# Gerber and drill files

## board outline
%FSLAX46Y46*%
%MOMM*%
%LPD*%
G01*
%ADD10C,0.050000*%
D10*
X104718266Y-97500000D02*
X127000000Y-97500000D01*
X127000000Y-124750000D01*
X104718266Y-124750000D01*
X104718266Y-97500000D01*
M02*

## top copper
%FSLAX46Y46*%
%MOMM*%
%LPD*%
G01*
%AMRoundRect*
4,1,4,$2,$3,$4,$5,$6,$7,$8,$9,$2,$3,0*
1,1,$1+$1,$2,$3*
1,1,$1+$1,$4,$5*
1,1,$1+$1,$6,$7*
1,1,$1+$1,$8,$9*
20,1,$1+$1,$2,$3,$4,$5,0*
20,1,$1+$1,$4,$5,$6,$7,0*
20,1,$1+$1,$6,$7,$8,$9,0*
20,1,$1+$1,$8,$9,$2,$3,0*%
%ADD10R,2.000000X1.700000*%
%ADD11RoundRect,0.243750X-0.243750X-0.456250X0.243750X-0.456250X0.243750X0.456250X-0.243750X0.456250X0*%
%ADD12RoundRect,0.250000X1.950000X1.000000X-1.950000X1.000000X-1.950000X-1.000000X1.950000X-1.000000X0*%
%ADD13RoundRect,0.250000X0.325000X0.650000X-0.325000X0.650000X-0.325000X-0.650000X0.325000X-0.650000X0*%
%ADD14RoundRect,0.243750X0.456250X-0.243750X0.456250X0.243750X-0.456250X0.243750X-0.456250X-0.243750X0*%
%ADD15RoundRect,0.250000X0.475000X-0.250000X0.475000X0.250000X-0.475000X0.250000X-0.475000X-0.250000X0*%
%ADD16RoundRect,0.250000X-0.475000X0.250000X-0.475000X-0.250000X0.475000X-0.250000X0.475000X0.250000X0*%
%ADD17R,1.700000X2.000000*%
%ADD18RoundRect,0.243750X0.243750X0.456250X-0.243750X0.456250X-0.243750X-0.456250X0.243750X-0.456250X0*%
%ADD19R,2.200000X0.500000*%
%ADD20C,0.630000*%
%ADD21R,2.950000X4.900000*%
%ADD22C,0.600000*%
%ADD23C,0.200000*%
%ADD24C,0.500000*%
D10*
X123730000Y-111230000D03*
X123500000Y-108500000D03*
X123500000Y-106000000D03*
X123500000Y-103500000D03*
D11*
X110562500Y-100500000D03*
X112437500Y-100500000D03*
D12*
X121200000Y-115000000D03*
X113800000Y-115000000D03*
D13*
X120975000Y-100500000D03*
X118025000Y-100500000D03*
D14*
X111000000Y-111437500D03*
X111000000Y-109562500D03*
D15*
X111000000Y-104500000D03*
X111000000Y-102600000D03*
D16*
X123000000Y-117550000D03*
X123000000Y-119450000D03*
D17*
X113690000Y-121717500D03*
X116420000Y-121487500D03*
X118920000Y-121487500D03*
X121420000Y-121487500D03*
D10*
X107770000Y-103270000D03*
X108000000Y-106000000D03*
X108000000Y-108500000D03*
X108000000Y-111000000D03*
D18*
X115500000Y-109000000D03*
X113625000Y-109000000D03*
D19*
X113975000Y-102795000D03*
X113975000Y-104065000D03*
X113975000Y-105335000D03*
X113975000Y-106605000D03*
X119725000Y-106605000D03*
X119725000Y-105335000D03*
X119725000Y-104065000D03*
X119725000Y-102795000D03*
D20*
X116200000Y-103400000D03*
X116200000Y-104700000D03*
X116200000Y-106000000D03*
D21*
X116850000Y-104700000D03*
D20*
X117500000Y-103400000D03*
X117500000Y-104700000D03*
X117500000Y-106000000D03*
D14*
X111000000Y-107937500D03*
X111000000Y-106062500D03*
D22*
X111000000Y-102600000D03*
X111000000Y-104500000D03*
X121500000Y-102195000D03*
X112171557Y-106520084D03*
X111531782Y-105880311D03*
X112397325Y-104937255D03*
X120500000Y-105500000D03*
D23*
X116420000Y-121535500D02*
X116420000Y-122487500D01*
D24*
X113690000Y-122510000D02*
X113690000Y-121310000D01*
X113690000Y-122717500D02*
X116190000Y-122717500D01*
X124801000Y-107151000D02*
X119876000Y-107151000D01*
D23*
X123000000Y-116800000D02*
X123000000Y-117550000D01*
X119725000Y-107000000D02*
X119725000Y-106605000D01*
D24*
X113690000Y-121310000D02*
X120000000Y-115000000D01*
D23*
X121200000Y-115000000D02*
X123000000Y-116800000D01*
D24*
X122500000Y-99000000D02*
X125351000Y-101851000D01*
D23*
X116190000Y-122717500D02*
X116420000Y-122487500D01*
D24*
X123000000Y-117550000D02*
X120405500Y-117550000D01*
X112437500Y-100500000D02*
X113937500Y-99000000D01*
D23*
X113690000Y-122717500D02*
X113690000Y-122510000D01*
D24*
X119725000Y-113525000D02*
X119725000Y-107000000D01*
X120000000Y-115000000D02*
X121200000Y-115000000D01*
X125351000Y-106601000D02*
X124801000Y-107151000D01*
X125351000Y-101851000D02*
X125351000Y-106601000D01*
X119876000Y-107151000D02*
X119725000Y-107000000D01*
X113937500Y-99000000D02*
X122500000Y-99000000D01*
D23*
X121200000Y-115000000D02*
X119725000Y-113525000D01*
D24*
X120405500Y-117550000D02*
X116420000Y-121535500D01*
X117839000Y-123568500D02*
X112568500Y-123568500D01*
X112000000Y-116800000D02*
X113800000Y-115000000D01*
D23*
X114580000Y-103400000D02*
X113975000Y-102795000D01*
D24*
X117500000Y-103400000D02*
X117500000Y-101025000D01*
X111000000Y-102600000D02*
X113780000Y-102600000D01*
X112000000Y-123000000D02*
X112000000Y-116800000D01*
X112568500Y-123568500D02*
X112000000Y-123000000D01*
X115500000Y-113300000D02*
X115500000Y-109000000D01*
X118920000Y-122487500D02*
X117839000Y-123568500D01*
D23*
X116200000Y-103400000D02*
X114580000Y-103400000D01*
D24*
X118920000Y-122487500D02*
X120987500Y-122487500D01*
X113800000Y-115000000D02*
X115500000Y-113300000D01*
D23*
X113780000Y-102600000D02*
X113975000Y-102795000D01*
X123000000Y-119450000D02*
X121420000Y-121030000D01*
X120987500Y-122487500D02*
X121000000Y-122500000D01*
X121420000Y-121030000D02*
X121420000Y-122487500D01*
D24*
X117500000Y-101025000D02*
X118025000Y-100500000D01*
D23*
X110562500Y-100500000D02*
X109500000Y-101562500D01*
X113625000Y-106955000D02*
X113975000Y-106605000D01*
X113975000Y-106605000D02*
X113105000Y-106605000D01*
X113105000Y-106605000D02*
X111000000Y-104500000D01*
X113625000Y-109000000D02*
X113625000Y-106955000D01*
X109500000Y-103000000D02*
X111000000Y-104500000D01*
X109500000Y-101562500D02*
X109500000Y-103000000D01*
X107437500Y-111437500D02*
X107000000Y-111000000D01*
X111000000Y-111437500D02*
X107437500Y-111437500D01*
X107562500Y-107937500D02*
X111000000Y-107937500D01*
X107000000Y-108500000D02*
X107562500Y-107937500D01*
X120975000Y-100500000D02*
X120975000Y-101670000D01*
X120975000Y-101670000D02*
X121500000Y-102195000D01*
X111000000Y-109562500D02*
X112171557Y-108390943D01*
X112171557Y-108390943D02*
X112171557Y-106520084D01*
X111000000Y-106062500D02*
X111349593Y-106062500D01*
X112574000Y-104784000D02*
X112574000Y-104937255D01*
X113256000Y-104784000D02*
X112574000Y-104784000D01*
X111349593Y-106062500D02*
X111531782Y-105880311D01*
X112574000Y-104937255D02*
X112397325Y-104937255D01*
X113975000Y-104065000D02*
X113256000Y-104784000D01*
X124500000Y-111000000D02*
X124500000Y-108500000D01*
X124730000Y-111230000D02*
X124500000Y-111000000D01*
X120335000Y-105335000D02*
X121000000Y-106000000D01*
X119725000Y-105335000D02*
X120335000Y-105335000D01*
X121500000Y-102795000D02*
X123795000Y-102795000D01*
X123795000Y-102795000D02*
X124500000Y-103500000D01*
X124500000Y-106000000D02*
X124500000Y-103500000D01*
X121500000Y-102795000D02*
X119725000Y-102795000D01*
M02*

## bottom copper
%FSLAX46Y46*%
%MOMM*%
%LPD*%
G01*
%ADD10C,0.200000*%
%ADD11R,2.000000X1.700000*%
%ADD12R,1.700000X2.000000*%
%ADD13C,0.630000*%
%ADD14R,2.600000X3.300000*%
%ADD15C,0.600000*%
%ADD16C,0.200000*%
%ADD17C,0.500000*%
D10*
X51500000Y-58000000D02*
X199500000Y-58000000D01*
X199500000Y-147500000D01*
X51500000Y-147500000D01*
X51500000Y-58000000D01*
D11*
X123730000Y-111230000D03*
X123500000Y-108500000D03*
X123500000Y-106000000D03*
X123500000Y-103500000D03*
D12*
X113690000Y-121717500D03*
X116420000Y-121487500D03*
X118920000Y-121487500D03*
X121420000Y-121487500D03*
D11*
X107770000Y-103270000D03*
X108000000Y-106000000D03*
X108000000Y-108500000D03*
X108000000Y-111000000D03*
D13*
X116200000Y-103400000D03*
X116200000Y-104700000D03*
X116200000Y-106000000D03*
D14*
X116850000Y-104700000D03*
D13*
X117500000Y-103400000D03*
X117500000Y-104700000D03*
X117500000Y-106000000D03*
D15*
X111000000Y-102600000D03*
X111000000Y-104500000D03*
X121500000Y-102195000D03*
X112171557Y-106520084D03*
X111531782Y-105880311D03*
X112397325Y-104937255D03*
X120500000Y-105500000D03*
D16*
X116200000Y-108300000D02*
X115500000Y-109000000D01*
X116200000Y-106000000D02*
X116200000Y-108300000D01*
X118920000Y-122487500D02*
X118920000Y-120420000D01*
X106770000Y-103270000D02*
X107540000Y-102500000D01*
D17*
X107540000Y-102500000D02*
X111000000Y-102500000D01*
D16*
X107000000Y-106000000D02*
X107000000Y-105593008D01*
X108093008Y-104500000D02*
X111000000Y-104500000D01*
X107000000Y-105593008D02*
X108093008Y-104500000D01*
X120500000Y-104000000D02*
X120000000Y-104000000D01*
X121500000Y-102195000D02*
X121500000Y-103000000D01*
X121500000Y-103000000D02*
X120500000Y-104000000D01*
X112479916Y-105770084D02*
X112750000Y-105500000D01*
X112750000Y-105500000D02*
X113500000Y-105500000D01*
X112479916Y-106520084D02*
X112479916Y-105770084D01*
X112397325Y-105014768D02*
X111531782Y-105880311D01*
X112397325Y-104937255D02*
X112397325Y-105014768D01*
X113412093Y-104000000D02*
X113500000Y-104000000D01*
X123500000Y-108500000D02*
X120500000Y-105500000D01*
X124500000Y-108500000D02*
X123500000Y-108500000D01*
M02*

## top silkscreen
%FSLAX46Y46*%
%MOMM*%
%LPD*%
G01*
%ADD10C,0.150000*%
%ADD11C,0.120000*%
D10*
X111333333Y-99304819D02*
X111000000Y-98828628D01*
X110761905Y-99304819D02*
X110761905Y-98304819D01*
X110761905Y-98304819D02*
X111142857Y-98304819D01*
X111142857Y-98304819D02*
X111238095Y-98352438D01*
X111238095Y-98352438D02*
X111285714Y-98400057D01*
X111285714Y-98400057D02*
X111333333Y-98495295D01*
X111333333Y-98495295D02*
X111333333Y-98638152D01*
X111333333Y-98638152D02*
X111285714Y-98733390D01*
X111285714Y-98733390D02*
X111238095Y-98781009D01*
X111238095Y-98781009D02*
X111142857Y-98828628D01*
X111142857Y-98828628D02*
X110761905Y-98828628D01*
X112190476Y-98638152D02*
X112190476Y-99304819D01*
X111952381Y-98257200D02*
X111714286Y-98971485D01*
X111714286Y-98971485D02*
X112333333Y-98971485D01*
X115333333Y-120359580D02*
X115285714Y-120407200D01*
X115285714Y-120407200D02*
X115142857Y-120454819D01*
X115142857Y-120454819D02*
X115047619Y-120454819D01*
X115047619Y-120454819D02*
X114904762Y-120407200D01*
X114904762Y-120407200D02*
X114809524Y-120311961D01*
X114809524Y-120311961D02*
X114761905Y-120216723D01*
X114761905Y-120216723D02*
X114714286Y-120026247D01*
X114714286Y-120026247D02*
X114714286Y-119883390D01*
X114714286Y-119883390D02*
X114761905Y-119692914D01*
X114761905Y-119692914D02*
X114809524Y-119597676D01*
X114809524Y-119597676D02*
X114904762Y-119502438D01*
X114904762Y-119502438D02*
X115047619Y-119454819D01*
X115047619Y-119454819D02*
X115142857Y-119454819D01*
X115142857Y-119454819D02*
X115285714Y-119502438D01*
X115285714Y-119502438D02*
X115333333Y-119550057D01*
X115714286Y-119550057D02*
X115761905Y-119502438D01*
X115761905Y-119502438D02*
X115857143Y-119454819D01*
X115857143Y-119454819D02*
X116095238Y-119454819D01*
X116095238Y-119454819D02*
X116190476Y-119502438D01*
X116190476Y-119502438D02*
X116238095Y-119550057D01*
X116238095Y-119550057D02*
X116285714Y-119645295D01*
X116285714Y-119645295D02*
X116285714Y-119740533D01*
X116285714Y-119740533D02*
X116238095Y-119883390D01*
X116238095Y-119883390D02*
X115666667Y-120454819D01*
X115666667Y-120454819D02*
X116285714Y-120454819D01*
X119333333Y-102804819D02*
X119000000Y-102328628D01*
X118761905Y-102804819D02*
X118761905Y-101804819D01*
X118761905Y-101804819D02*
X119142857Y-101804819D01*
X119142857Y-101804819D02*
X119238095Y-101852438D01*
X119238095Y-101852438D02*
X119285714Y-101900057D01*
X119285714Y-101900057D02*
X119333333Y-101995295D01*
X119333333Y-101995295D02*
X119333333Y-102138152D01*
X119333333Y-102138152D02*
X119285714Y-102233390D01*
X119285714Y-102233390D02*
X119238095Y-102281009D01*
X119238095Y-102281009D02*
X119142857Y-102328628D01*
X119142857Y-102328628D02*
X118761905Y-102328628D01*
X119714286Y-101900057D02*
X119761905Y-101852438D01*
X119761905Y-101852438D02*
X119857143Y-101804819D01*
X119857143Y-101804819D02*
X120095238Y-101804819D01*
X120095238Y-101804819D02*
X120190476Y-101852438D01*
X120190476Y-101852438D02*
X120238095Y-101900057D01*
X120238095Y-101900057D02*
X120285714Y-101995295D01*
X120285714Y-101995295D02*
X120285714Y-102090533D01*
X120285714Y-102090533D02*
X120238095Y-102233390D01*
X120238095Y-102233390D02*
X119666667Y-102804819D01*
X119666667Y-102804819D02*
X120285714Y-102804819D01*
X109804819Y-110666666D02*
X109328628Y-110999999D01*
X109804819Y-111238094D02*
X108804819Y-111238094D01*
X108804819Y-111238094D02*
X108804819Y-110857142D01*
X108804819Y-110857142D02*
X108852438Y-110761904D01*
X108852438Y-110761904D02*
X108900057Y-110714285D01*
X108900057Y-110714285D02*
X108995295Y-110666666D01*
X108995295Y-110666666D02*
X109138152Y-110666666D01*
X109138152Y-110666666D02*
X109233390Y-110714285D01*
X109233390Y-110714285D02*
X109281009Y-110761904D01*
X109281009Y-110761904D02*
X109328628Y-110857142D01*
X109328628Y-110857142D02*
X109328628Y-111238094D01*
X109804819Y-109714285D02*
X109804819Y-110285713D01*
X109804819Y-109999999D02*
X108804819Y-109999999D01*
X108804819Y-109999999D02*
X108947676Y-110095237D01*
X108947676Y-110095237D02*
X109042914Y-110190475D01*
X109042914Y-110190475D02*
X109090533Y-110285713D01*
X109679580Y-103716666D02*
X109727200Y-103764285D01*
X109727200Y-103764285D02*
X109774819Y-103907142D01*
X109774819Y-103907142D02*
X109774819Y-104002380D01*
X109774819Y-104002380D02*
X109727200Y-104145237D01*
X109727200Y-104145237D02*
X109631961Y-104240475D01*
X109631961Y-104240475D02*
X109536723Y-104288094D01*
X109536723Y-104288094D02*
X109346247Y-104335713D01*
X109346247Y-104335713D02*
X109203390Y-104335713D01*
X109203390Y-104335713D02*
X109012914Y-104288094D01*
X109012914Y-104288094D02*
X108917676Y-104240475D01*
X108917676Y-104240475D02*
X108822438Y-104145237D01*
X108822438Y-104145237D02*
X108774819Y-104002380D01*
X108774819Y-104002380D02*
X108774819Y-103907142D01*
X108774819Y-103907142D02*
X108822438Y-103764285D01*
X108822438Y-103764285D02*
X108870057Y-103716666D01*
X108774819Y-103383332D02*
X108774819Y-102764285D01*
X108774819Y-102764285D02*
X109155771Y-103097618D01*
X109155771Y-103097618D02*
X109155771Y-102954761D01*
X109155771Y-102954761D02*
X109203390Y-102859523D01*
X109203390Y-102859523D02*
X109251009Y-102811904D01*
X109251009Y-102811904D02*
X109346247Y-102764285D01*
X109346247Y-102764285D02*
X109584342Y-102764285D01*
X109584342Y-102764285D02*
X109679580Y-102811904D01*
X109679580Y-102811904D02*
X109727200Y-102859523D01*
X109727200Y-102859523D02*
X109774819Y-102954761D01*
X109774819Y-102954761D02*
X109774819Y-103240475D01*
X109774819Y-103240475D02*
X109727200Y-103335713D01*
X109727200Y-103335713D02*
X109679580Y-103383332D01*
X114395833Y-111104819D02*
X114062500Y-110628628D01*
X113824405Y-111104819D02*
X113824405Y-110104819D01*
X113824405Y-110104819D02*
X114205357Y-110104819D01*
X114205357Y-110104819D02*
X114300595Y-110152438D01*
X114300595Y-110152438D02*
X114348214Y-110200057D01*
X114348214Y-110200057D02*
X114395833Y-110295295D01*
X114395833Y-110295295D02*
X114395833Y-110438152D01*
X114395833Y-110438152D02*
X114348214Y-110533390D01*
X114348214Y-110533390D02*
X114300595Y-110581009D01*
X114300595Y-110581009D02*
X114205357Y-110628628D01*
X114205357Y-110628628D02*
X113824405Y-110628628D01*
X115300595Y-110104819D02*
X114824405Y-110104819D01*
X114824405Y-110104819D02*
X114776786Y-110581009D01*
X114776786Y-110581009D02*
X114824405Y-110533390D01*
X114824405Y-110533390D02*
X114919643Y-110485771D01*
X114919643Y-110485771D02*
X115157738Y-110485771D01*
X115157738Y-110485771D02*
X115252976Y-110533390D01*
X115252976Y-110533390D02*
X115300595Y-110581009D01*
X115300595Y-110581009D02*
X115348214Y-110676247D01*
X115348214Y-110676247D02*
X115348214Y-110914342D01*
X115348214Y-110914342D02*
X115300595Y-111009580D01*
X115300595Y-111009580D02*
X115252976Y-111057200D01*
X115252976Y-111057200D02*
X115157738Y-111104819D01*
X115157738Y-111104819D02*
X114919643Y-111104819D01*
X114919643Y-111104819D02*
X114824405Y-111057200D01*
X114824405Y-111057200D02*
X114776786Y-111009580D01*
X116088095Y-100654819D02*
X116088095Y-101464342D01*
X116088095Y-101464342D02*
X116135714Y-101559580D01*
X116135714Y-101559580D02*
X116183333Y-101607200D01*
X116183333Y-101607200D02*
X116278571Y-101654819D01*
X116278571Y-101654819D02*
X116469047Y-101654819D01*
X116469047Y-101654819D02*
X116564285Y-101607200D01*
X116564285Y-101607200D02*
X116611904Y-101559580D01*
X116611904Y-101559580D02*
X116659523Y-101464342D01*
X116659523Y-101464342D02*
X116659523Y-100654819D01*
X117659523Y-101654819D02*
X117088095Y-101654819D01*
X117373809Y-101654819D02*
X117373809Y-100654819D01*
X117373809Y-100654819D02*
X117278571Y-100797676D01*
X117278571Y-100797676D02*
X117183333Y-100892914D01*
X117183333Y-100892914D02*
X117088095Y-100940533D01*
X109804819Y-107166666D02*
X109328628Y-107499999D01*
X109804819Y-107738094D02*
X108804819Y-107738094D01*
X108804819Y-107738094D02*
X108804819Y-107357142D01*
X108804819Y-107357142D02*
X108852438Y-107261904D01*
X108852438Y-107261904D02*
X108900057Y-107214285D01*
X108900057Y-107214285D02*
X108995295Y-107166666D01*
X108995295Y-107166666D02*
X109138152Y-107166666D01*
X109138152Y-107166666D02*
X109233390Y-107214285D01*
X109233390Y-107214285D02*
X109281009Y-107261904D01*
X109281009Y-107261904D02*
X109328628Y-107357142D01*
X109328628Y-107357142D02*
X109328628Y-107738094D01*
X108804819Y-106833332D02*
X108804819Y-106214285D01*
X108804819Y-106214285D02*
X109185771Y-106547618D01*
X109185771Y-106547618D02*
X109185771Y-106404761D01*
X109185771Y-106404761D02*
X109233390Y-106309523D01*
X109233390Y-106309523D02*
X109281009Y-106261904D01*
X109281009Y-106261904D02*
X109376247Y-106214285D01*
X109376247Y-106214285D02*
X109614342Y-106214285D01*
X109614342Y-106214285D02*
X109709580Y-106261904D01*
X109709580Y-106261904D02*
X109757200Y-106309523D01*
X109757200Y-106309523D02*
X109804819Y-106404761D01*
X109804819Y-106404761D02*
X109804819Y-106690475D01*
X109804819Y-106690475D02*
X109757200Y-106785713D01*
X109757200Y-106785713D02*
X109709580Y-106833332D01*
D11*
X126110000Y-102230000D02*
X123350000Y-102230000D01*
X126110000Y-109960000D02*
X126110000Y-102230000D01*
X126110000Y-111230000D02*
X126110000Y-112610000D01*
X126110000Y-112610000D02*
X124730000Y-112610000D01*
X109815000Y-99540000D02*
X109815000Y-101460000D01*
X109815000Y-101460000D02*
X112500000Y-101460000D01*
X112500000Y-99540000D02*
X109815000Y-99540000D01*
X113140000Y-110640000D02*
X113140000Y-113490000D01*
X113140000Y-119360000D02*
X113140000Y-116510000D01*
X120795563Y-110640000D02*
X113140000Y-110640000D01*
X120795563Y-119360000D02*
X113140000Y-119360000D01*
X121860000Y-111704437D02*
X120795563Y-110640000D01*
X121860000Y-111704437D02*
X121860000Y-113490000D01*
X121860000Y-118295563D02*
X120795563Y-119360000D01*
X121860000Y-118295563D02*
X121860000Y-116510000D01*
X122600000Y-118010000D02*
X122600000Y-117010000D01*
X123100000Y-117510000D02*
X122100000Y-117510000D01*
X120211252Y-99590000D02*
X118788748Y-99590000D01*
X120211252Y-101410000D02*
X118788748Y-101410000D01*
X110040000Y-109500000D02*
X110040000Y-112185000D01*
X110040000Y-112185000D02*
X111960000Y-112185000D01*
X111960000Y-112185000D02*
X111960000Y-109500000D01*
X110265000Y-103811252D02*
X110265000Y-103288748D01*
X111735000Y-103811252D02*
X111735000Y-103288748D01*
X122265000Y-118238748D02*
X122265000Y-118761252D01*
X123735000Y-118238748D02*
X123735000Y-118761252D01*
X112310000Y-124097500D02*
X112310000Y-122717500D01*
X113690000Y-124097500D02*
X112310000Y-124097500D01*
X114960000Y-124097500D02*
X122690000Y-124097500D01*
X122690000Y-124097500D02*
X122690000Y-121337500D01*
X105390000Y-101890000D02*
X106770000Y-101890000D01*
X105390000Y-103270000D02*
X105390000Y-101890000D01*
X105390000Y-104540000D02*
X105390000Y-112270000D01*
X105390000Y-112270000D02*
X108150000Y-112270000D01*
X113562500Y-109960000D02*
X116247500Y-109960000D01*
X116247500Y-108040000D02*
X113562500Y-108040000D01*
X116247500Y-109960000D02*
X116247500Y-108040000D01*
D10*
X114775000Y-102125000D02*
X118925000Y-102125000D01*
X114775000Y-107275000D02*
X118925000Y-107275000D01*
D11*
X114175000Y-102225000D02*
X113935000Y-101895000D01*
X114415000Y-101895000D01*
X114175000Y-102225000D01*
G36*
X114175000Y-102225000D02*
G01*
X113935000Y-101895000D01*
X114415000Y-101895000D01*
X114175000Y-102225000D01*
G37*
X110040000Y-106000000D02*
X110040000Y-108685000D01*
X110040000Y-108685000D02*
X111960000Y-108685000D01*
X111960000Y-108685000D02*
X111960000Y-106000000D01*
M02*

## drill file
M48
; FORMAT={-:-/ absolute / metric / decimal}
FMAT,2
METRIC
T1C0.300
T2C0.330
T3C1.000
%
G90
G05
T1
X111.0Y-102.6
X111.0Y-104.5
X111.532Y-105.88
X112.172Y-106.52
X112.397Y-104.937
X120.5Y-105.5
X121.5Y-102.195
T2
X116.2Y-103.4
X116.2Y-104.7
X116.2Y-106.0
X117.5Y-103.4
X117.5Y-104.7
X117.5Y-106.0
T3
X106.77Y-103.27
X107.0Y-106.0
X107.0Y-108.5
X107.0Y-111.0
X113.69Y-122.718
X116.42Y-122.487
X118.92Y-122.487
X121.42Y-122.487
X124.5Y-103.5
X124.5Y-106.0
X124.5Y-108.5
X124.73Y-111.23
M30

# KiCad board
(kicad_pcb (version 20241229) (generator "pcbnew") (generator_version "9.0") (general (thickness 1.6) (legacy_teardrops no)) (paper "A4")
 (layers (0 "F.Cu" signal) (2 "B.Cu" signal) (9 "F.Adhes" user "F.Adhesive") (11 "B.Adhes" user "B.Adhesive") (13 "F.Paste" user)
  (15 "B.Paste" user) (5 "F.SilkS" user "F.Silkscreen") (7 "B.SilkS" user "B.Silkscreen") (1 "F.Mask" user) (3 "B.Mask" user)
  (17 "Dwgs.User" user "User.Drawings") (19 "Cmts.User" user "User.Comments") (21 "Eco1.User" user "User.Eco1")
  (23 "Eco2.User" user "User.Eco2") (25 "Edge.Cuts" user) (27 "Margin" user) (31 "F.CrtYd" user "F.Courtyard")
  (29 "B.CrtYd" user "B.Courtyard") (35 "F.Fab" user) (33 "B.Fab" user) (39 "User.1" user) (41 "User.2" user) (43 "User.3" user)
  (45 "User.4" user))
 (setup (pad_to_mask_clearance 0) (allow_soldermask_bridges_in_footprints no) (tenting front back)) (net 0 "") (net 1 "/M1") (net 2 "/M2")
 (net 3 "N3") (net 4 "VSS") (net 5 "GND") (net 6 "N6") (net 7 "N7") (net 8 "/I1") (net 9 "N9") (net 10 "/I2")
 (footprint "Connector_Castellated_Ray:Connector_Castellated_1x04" (layer "F.Cu") (at 123.5 108.5 180)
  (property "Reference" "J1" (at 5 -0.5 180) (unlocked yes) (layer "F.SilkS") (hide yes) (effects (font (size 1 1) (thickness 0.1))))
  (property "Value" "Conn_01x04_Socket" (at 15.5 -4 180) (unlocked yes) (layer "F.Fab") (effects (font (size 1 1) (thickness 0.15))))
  (fp_line (start -2.61 6.27) (end 0.15 6.27) (stroke (width 0.12) (type solid)) (layer "F.SilkS"))
  (fp_line (start -2.61 -1.46) (end -2.61 6.27) (stroke (width 0.12) (type solid)) (layer "F.SilkS"))
  (fp_line (start -2.61 -2.73) (end -2.61 -4.11) (stroke (width 0.12) (type solid)) (layer "F.SilkS"))
  (fp_line (start -2.61 -4.11) (end -1.23 -4.11) (stroke (width 0.12) (type solid)) (layer "F.SilkS"))
  (pad "1" thru_hole rect (at -1.23 -2.73 180) (size 2 1.7) (drill 1 (offset 1 0)) (layers "*.Cu" "*.Mask") (remove_unused_layers no)
   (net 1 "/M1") (solder_mask_margin 0.04))
  (pad "2" thru_hole rect (at -1 0 180) (size 2 1.7) (drill 1 (offset 1 0)) (layers "*.Cu" "*.Mask") (remove_unused_layers no) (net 1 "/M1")
   (solder_mask_margin 0.04))
  (pad "3" thru_hole rect (at -1 2.5 180) (size 2 1.7) (drill 1 (offset 1 0)) (layers "*.Cu" "*.Mask") (remove_unused_layers no)
   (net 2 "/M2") (solder_mask_margin 0.04))
  (pad "4" thru_hole rect (at -1 5 180) (size 2 1.7) (drill 1 (offset 1 0)) (layers "*.Cu" "*.Mask") (remove_unused_layers no) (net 2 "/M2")
   (solder_mask_margin 0.04)))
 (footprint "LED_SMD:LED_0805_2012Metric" (layer "F.Cu") (at 111.5 100.5)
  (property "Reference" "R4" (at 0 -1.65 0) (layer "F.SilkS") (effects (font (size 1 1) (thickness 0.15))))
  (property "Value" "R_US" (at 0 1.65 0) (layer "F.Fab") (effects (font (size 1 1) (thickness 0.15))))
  (fp_line (start -1.685 -0.96) (end -1.685 0.96) (stroke (width 0.12) (type solid)) (layer "F.SilkS"))
  (fp_line (start -1.685 0.96) (end 1 0.96) (stroke (width 0.12) (type solid)) (layer "F.SilkS"))
  (fp_line (start 1 -0.96) (end -1.685 -0.96) (stroke (width 0.12) (type solid)) (layer "F.SilkS"))
  (pad "1" smd roundrect (at -0.9375 0) (size 0.975 1.4) (layers "F.Cu" "F.Mask" "F.Paste") (roundrect_rratio 0.25) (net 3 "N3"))
  (pad "2" smd roundrect (at 0.9375 0) (size 0.975 1.4) (layers "F.Cu" "F.Mask" "F.Paste") (roundrect_rratio 0.25) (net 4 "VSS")))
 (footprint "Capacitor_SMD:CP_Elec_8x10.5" (layer "F.Cu") (at 117.5 115 180)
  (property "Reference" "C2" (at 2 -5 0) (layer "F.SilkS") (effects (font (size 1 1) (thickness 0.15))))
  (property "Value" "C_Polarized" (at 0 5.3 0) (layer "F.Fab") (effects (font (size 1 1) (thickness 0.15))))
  (fp_line (start 4.36 4.36) (end 4.36 1.51) (stroke (width 0.12) (type solid)) (layer "F.SilkS"))
  (fp_line (start 4.36 -4.36) (end 4.36 -1.51) (stroke (width 0.12) (type solid)) (layer "F.SilkS"))
  (fp_line (start -3.295563 4.36) (end 4.36 4.36) (stroke (width 0.12) (type solid)) (layer "F.SilkS"))
  (fp_line (start -3.295563 -4.36) (end 4.36 -4.36) (stroke (width 0.12) (type solid)) (layer "F.SilkS"))
  (fp_line (start -4.36 3.295563) (end -3.295563 4.36) (stroke (width 0.12) (type solid)) (layer "F.SilkS"))
  (fp_line (start -4.36 3.295563) (end -4.36 1.51) (stroke (width 0.12) (type solid)) (layer "F.SilkS"))
  (fp_line (start -4.36 -3.295563) (end -3.295563 -4.36) (stroke (width 0.12) (type solid)) (layer "F.SilkS"))
  (fp_line (start -4.36 -3.295563) (end -4.36 -1.51) (stroke (width 0.12) (type solid)) (layer "F.SilkS"))
  (fp_line (start -5.1 -3.01) (end -5.1 -2.01) (stroke (width 0.12) (type solid)) (layer "F.SilkS"))
  (fp_line (start -5.6 -2.51) (end -4.6 -2.51) (stroke (width 0.12) (type solid)) (layer "F.SilkS"))
  (pad "1" smd roundrect (at -3.7 0 180) (size 4.4 2.5) (layers "F.Cu" "F.Mask" "F.Paste") (roundrect_rratio 0.1) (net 4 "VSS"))
  (pad "2" smd roundrect (at 3.7 0 180) (size 4.4 2.5) (layers "F.Cu" "F.Mask" "F.Paste") (roundrect_rratio 0.1) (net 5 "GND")))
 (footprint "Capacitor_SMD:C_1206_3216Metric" (layer "F.Cu") (at 119.5 100.5 180)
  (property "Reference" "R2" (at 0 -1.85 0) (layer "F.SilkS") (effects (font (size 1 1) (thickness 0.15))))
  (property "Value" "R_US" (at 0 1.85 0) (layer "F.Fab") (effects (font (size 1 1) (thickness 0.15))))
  (fp_line (start -0.711252 0.91) (end 0.711252 0.91) (stroke (width 0.12) (type solid)) (layer "F.SilkS"))
  (fp_line (start -0.711252 -0.91) (end 0.711252 -0.91) (stroke (width 0.12) (type solid)) (layer "F.SilkS"))
  (pad "1" smd roundrect (at -1.475 0 180) (size 1.15 1.8) (layers "F.Cu" "F.Mask" "F.Paste") (roundrect_rratio 0.217391) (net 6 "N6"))
  (pad "2" smd roundrect (at 1.475 0 180) (size 1.15 1.8) (layers "F.Cu" "F.Mask" "F.Paste") (roundrect_rratio 0.217391) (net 5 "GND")))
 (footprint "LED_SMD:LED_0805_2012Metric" (layer "F.Cu") (at 111 110.5 90)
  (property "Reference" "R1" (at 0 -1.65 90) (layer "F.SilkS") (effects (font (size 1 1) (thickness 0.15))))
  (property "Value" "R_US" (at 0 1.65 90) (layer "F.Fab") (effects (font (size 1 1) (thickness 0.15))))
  (fp_line (start 1 -0.96) (end -1.685 -0.96) (stroke (width 0.12) (type solid)) (layer "F.SilkS"))
  (fp_line (start -1.685 -0.96) (end -1.685 0.96) (stroke (width 0.12) (type solid)) (layer "F.SilkS"))
  (fp_line (start -1.685 0.96) (end 1 0.96) (stroke (width 0.12) (type solid)) (layer "F.SilkS"))
  (pad "1" smd roundrect (at -0.9375 0 90) (size 0.975 1.4) (layers "F.Cu" "F.Mask" "F.Paste") (roundrect_rratio 0.25) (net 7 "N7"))
  (pad "2" smd roundrect (at 0.9375 0 90) (size 0.975 1.4) (layers "F.Cu" "F.Mask" "F.Paste") (roundrect_rratio 0.25) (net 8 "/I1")))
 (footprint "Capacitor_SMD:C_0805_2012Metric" (layer "F.Cu") (at 111 103.55 90)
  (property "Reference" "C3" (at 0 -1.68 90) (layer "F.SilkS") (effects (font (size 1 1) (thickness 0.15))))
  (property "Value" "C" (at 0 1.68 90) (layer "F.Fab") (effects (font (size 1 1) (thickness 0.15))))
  (fp_line (start -0.261252 -0.735) (end 0.261252 -0.735) (stroke (width 0.12) (type solid)) (layer "F.SilkS"))
  (fp_line (start -0.261252 0.735) (end 0.261252 0.735) (stroke (width 0.12) (type solid)) (layer "F.SilkS"))
  (pad "1" smd roundrect (at -0.95 0 90) (size 1 1.45) (layers "F.Cu" "F.Mask" "F.Paste") (roundrect_rratio 0.25) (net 3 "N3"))
  (pad "2" smd roundrect (at 0.95 0 90) (size 1 1.45) (layers "F.Cu" "F.Mask" "F.Paste") (roundrect_rratio 0.25) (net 5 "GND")))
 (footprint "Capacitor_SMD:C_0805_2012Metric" (layer "F.Cu") (at 123 118.5 -90)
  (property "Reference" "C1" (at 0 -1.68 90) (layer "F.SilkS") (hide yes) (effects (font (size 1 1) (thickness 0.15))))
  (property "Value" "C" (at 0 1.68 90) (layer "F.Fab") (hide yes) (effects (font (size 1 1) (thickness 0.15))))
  (fp_line (start -0.261252 0.735) (end 0.261252 0.735) (stroke (width 0.12) (type solid)) (layer "F.SilkS"))
  (fp_line (start -0.261252 -0.735) (end 0.261252 -0.735) (stroke (width 0.12) (type solid)) (layer "F.SilkS"))
  (pad "1" smd roundrect (at -0.95 0 270) (size 1 1.45) (layers "F.Cu" "F.Mask" "F.Paste") (roundrect_rratio 0.25) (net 4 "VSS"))
  (pad "2" smd roundrect (at 0.95 0 270) (size 1 1.45) (layers "F.Cu" "F.Mask" "F.Paste") (roundrect_rratio 0.25) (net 5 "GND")))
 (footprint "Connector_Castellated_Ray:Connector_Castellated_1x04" (layer "F.Cu") (at 116.42 121.4875 90)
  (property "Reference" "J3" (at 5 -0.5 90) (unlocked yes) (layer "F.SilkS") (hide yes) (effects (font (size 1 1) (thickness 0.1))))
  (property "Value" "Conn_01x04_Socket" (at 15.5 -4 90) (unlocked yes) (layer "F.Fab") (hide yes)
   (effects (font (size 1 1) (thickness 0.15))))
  (fp_line (start -2.61 -4.11) (end -1.23 -4.11) (stroke (width 0.12) (type solid)) (layer "F.SilkS"))
  (fp_line (start -2.61 -2.73) (end -2.61 -4.11) (stroke (width 0.12) (type solid)) (layer "F.SilkS"))
  (fp_line (start -2.61 -1.46) (end -2.61 6.27) (stroke (width 0.12) (type solid)) (layer "F.SilkS"))
  (fp_line (start -2.61 6.27) (end 0.15 6.27) (stroke (width 0.12) (type solid)) (layer "F.SilkS"))
  (pad "1" thru_hole rect (at -1.23 -2.73 90) (size 2 1.7) (drill 1 (offset 1 0)) (layers "*.Cu" "*.Mask") (remove_unused_layers no)
   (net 4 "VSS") (solder_mask_margin 0.04))
  (pad "2" thru_hole rect (at -1 0 90) (size 2 1.7) (drill 1 (offset 1 0)) (layers "*.Cu" "*.Mask") (remove_unused_layers no) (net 4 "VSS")
   (solder_mask_margin 0.04))
  (pad "3" thru_hole rect (at -1 2.5 90) (size 2 1.7) (drill 1 (offset 1 0)) (layers "*.Cu" "*.Mask") (remove_unused_layers no)
   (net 5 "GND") (solder_mask_margin 0.04))
  (pad "4" thru_hole rect (at -1 5 90) (size 2 1.7) (drill 1 (offset 1 0)) (layers "*.Cu" "*.Mask") (remove_unused_layers no) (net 5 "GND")
   (solder_mask_margin 0.04)))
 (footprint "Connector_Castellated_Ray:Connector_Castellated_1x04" (layer "F.Cu") (at 108 106)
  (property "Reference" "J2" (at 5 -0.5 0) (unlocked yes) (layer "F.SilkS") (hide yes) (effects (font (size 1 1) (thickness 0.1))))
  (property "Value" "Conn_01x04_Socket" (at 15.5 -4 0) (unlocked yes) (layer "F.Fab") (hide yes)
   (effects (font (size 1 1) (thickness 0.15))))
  (fp_line (start -2.61 -4.11) (end -1.23 -4.11) (stroke (width 0.12) (type solid)) (layer "F.SilkS"))
  (fp_line (start -2.61 -2.73) (end -2.61 -4.11) (stroke (width 0.12) (type solid)) (layer "F.SilkS"))
  (fp_line (start -2.61 -1.46) (end -2.61 6.27) (stroke (width 0.12) (type solid)) (layer "F.SilkS"))
  (fp_line (start -2.61 6.27) (end 0.15 6.27) (stroke (width 0.12) (type solid)) (layer "F.SilkS"))
  (pad "1" thru_hole rect (at -1.23 -2.73) (size 2 1.7) (drill 1 (offset 1 0)) (layers "*.Cu" "*.Mask") (remove_unused_layers no)
   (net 5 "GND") (solder_mask_margin 0.04))
  (pad "2" thru_hole rect (at -1 0) (size 2 1.7) (drill 1 (offset 1 0)) (layers "*.Cu" "*.Mask") (remove_unused_layers no) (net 3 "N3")
   (solder_mask_margin 0.04))
  (pad "3" thru_hole rect (at -1 2.5) (size 2 1.7) (drill 1 (offset 1 0)) (layers "*.Cu" "*.Mask") (remove_unused_layers no) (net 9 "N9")
   (solder_mask_margin 0.04))
  (pad "4" thru_hole rect (at -1 5) (size 2 1.7) (drill 1 (offset 1 0)) (layers "*.Cu" "*.Mask") (remove_unused_layers no) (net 7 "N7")
   (solder_mask_margin 0.04)))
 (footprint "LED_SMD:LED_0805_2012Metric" (layer "F.Cu") (at 114.5625 109 180)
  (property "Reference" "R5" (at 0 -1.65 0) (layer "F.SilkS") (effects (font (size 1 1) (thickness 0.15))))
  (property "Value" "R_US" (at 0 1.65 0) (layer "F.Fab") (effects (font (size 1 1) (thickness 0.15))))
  (fp_line (start 1 -0.96) (end -1.685 -0.96) (stroke (width 0.12) (type solid)) (layer "F.SilkS"))
  (fp_line (start -1.685 0.96) (end 1 0.96) (stroke (width 0.12) (type solid)) (layer "F.SilkS"))
  (fp_line (start -1.685 -0.96) (end -1.685 0.96) (stroke (width 0.12) (type solid)) (layer "F.SilkS"))
  (pad "1" smd roundrect (at -0.9375 0 180) (size 0.975 1.4) (layers "F.Cu" "F.Mask" "F.Paste") (roundrect_rratio 0.25) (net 5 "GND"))
  (pad "2" smd roundrect (at 0.9375 0 180) (size 0.975 1.4) (layers "F.Cu" "F.Mask" "F.Paste") (roundrect_rratio 0.25) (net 3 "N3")))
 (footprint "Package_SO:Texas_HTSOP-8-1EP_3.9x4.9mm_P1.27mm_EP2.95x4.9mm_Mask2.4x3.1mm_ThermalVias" (layer "F.Cu") (at 116.85 104.7)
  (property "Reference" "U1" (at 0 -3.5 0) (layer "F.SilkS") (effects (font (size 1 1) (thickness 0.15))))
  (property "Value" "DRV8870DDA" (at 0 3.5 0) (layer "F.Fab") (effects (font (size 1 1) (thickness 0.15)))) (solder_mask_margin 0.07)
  (fp_line (start -2.075 -2.575) (end 2.075 -2.575) (stroke (width 0.15) (type solid)) (layer "F.SilkS"))
  (fp_line (start -2.075 2.575) (end 2.075 2.575) (stroke (width 0.15) (type solid)) (layer "F.SilkS"))
  (fp_poly
   (pts (xy -2.675 -2.475) (xy -2.915 -2.805) (xy -2.435 -2.805) (xy -2.675 -2.475)) (stroke (width 0.12) (type solid)) (fill yes)
   (layer "F.SilkS"))
  (pad "" smd rect (at 0 0) (size 2.4 3.1) (layers "F.Mask")) (pad "" smd rect (at 0 0) (size 2.4 3.1) (layers "F.Paste"))
  (pad "1" smd rect (at -2.875 -1.905) (size 2.2 0.5) (layers "F.Cu" "F.Mask" "F.Paste") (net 5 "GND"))
  (pad "2" smd rect (at -2.875 -0.635) (size 2.2 0.5) (layers "F.Cu" "F.Mask" "F.Paste") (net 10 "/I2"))
  (pad "3" smd rect (at -2.875 0.635) (size 2.2 0.5) (layers "F.Cu" "F.Mask" "F.Paste") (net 8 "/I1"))
  (pad "4" smd rect (at -2.875 1.905) (size 2.2 0.5) (layers "F.Cu" "F.Mask" "F.Paste") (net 3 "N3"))
  (pad "5" smd rect (at 2.875 1.905) (size 2.2 0.5) (layers "F.Cu" "F.Mask" "F.Paste") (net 4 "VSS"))
  (pad "6" smd rect (at 2.875 0.635) (size 2.2 0.5) (layers "F.Cu" "F.Mask" "F.Paste") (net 1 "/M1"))
  (pad "7" smd rect (at 2.875 -0.635) (size 2.2 0.5) (layers "F.Cu" "F.Mask" "F.Paste") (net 6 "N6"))
  (pad "8" smd rect (at 2.875 -1.905) (size 2.2 0.5) (layers "F.Cu" "F.Mask" "F.Paste") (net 2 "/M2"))
  (pad "9" thru_hole circle (at -0.65 -1.3) (size 0.63 0.63) (drill 0.33) (layers "*.Cu" "*.Mask") (remove_unused_layers no) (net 5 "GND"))
  (pad "9" thru_hole circle (at -0.65 0) (size 0.63 0.63) (drill 0.33) (layers "*.Cu" "*.Mask") (remove_unused_layers no) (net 5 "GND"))
  (pad "9" thru_hole circle (at -0.65 1.3) (size 0.63 0.63) (drill 0.33) (layers "*.Cu" "*.Mask") (remove_unused_layers no) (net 5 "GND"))
  (pad "9" smd rect (at 0 0) (size 2.6 3.3) (layers "B.Cu") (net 5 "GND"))
  (pad "9" smd rect (at 0 0) (size 2.95 4.9) (layers "F.Cu") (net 5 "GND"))
  (pad "9" thru_hole circle (at 0.65 -1.3) (size 0.63 0.63) (drill 0.33) (layers "*.Cu" "*.Mask") (remove_unused_layers no) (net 5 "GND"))
  (pad "9" thru_hole circle (at 0.65 0) (size 0.63 0.63) (drill 0.33) (layers "*.Cu" "*.Mask") (remove_unused_layers no) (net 5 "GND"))
  (pad "9" thru_hole circle (at 0.65 1.3) (size 0.63 0.63) (drill 0.33) (layers "*.Cu" "*.Mask") (remove_unused_layers no) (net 5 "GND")))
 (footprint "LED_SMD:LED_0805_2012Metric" (layer "F.Cu") (at 111 107 90)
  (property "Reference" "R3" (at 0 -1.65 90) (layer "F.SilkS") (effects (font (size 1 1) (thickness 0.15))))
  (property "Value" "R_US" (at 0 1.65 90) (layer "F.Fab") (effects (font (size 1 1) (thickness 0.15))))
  (fp_line (start 1 -0.96) (end -1.685 -0.96) (stroke (width 0.12) (type solid)) (layer "F.SilkS"))
  (fp_line (start -1.685 -0.96) (end -1.685 0.96) (stroke (width 0.12) (type solid)) (layer "F.SilkS"))
  (fp_line (start -1.685 0.96) (end 1 0.96) (stroke (width 0.12) (type solid)) (layer "F.SilkS"))
  (pad "1" smd roundrect (at -0.9375 0 90) (size 0.975 1.4) (layers "F.Cu" "F.Mask" "F.Paste") (roundrect_rratio 0.25) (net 9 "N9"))
  (pad "2" smd roundrect (at 0.9375 0 90) (size 0.975 1.4) (layers "F.Cu" "F.Mask" "F.Paste") (roundrect_rratio 0.25) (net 10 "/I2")))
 (gr_rect (start 51.5 58) (end 199.5 147.5) (stroke (width 0.2) (type default)) (fill no) (layer "B.Cu"))
 (gr_rect (start 104.718266 97.5) (end 127 124.75) (stroke (width 0.05) (type default)) (fill no) (layer "Edge.Cuts"))
 (segment (start 116.42 121.5355) (end 116.42 122.4875) (width 0.2) (layer "F.Cu") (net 4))
 (segment (start 113.69 122.51) (end 113.69 121.31) (width 0.5) (layer "F.Cu") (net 4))
 (segment (start 113.69 122.7175) (end 116.19 122.7175) (width 0.5) (layer "F.Cu") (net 4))
 (segment (start 124.801 107.151) (end 119.876 107.151) (width 0.5) (layer "F.Cu") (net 4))
 (segment (start 123 116.8) (end 123 117.55) (width 0.2) (layer "F.Cu") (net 4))
 (segment (start 119.725 107) (end 119.725 106.605) (width 0.2) (layer "F.Cu") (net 4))
 (segment (start 113.69 121.31) (end 120 115) (width 0.5) (layer "F.Cu") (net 4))
 (segment (start 121.2 115) (end 123 116.8) (width 0.2) (layer "F.Cu") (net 4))
 (segment (start 122.5 99) (end 125.351 101.851) (width 0.5) (layer "F.Cu") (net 4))
 (segment (start 116.19 122.7175) (end 116.42 122.4875) (width 0.2) (layer "F.Cu") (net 4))
 (segment (start 123 117.55) (end 120.4055 117.55) (width 0.5) (layer "F.Cu") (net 4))
 (segment (start 112.4375 100.5) (end 113.9375 99) (width 0.5) (layer "F.Cu") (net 4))
 (segment (start 113.69 122.7175) (end 113.69 122.51) (width 0.2) (layer "F.Cu") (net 4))
 (segment (start 119.725 113.525) (end 119.725 107) (width 0.5) (layer "F.Cu") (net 4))
 (segment (start 120 115) (end 121.2 115) (width 0.5) (layer "F.Cu") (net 4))
 (segment (start 125.351 106.601) (end 124.801 107.151) (width 0.5) (layer "F.Cu") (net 4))
 (segment (start 125.351 101.851) (end 125.351 106.601) (width 0.5) (layer "F.Cu") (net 4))
 (segment (start 119.876 107.151) (end 119.725 107) (width 0.5) (layer "F.Cu") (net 4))
 (segment (start 113.9375 99) (end 122.5 99) (width 0.5) (layer "F.Cu") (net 4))
 (segment (start 121.2 115) (end 119.725 113.525) (width 0.2) (layer "F.Cu") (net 4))
 (segment (start 120.4055 117.55) (end 116.42 121.5355) (width 0.5) (layer "F.Cu") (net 4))
 (segment (start 117.839 123.5685) (end 112.5685 123.5685) (width 0.5) (layer "F.Cu") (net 5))
 (segment (start 112 116.8) (end 113.8 115) (width 0.5) (layer "F.Cu") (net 5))
 (segment (start 114.58 103.4) (end 113.975 102.795) (width 0.2) (layer "F.Cu") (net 5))
 (segment (start 117.5 103.4) (end 117.5 101.025) (width 0.5) (layer "F.Cu") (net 5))
 (segment (start 111 102.6) (end 113.78 102.6) (width 0.5) (layer "F.Cu") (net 5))
 (segment (start 112 123) (end 112 116.8) (width 0.5) (layer "F.Cu") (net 5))
 (segment (start 112.5685 123.5685) (end 112 123) (width 0.5) (layer "F.Cu") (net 5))
 (segment (start 115.5 113.3) (end 115.5 109) (width 0.5) (layer "F.Cu") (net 5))
 (segment (start 118.92 122.4875) (end 117.839 123.5685) (width 0.5) (layer "F.Cu") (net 5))
 (segment (start 116.2 103.4) (end 114.58 103.4) (width 0.2) (layer "F.Cu") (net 5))
 (segment (start 118.92 122.4875) (end 120.9875 122.4875) (width 0.5) (layer "F.Cu") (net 5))
 (segment (start 113.8 115) (end 115.5 113.3) (width 0.5) (layer "F.Cu") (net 5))
 (segment (start 113.78 102.6) (end 113.975 102.795) (width 0.2) (layer "F.Cu") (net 5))
 (segment (start 123 119.45) (end 121.42 121.03) (width 0.2) (layer "F.Cu") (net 5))
 (segment (start 120.9875 122.4875) (end 121 122.5) (width 0.2) (layer "F.Cu") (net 5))
 (segment (start 121.42 121.03) (end 121.42 122.4875) (width 0.2) (layer "F.Cu") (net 5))
 (segment (start 117.5 101.025) (end 118.025 100.5) (width 0.5) (layer "F.Cu") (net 5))
 (via (at 111 102.6) (size 0.6) (drill 0.3) (layers "F.Cu" "B.Cu") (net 5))
 (segment (start 116.2 108.3) (end 115.5 109) (width 0.2) (layer "B.Cu") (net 5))
 (segment (start 116.2 106) (end 116.2 108.3) (width 0.2) (layer "B.Cu") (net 5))
 (segment (start 118.92 122.4875) (end 118.92 120.42) (width 0.2) (layer "B.Cu") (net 5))
 (segment (start 106.77 103.27) (end 107.54 102.5) (width 0.2) (layer "B.Cu") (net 5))
 (segment (start 107.54 102.5) (end 111 102.5) (width 0.5) (layer "B.Cu") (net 5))
 (segment (start 110.5625 100.5) (end 109.5 101.5625) (width 0.2) (layer "F.Cu") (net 3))
 (segment (start 113.625 106.955) (end 113.975 106.605) (width 0.2) (layer "F.Cu") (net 3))
 (segment (start 113.975 106.605) (end 113.105 106.605) (width 0.2) (layer "F.Cu") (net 3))
 (segment (start 113.105 106.605) (end 111 104.5) (width 0.2) (layer "F.Cu") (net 3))
 (segment (start 113.625 109) (end 113.625 106.955) (width 0.2) (layer "F.Cu") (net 3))
 (segment (start 109.5 103) (end 111 104.5) (width 0.2) (layer "F.Cu") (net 3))
 (segment (start 109.5 101.5625) (end 109.5 103) (width 0.2) (layer "F.Cu") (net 3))
 (via (at 111 104.5) (size 0.6) (drill 0.3) (layers "F.Cu" "B.Cu") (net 3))
 (segment (start 107 106) (end 107 105.593008) (width 0.2) (layer "B.Cu") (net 3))
 (segment (start 108.093008 104.5) (end 111 104.5) (width 0.2) (layer "B.Cu") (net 3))
 (segment (start 107 105.593008) (end 108.093008 104.5) (width 0.2) (layer "B.Cu") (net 3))
 (segment (start 107.4375 111.4375) (end 107 111) (width 0.2) (layer "F.Cu") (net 7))
 (segment (start 111 111.4375) (end 107.4375 111.4375) (width 0.2) (layer "F.Cu") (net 7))
 (segment (start 107.5625 107.9375) (end 111 107.9375) (width 0.2) (layer "F.Cu") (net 9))
 (segment (start 107 108.5) (end 107.5625 107.9375) (width 0.2) (layer "F.Cu") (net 9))
 (segment (start 120.975 100.5) (end 120.975 101.67) (width 0.2) (layer "F.Cu") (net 6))
 (segment (start 120.975 101.67) (end 121.5 102.195) (width 0.2) (layer "F.Cu") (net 6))
 (via (at 121.5 102.195) (size 0.6) (drill 0.3) (layers "F.Cu" "B.Cu") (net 6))
 (segment (start 120.5 104) (end 120 104) (width 0.2) (layer "B.Cu") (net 6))
 (segment (start 121.5 102.195) (end 121.5 103) (width 0.2) (layer "B.Cu") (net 6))
 (segment (start 121.5 103) (end 120.5 104) (width 0.2) (layer "B.Cu") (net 6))
 (segment (start 111 109.5625) (end 112.171557 108.390943) (width 0.2) (layer "F.Cu") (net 8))
 (segment (start 112.171557 108.390943) (end 112.171557 106.520084) (width 0.2) (layer "F.Cu") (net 8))
 (via (at 112.171557 106.520084) (size 0.6) (drill 0.3) (layers "F.Cu" "B.Cu") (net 8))
 (segment (start 112.479916 105.770084) (end 112.75 105.5) (width 0.2) (layer "B.Cu") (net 8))
 (segment (start 112.75 105.5) (end 113.5 105.5) (width 0.2) (layer "B.Cu") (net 8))
 (segment (start 112.479916 106.520084) (end 112.479916 105.770084) (width 0.2) (layer "B.Cu") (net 8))
 (segment (start 111 106.0625) (end 111.349593 106.0625) (width 0.2) (layer "F.Cu") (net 10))
 (segment (start 112.574 104.784) (end 112.574 104.937255) (width 0.2) (layer "F.Cu") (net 10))
 (segment (start 113.256 104.784) (end 112.574 104.784) (width 0.2) (layer "F.Cu") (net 10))
 (segment (start 111.349593 106.0625) (end 111.531782 105.880311) (width 0.2) (layer "F.Cu") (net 10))
 (segment (start 112.574 104.937255) (end 112.397325 104.937255) (width 0.2) (layer "F.Cu") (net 10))
 (segment (start 113.975 104.065) (end 113.256 104.784) (width 0.2) (layer "F.Cu") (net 10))
 (via (at 111.531782 105.880311) (size 0.6) (drill 0.3) (layers "F.Cu" "B.Cu") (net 10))
 (via (at 112.397325 104.937255) (size 0.6) (drill 0.3) (layers "F.Cu" "B.Cu") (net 10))
 (segment (start 112.397325 105.014768) (end 111.531782 105.880311) (width 0.2) (layer "B.Cu") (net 10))
 (segment (start 112.397325 104.937255) (end 112.397325 105.014768) (width 0.2) (layer "B.Cu") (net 10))
 (segment (start 113.412093 104) (end 113.5 104) (width 0.2) (layer "B.Cu") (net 10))
 (segment (start 124.5 111) (end 124.5 108.5) (width 0.2) (layer "F.Cu") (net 1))
 (segment (start 124.73 111.23) (end 124.5 111) (width 0.2) (layer "F.Cu") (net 1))
 (segment (start 120.335 105.335) (end 121 106) (width 0.2) (layer "F.Cu") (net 1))
 (segment (start 119.725 105.335) (end 120.335 105.335) (width 0.2) (layer "F.Cu") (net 1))
 (via (at 120.5 105.5) (size 0.6) (drill 0.3) (layers "F.Cu" "B.Cu") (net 1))
 (segment (start 123.5 108.5) (end 120.5 105.5) (width 0.2) (layer "B.Cu") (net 1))
 (segment (start 124.5 108.5) (end 123.5 108.5) (width 0.2) (layer "B.Cu") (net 1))
 (segment (start 121.5 102.795) (end 123.795 102.795) (width 0.2) (layer "F.Cu") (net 2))
 (segment (start 123.795 102.795) (end 124.5 103.5) (width 0.2) (layer "F.Cu") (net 2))
 (segment (start 124.5 106) (end 124.5 103.5) (width 0.2) (layer "F.Cu") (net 2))
 (segment (start 121.5 102.795) (end 119.725 102.795) (width 0.2) (layer "F.Cu") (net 2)))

